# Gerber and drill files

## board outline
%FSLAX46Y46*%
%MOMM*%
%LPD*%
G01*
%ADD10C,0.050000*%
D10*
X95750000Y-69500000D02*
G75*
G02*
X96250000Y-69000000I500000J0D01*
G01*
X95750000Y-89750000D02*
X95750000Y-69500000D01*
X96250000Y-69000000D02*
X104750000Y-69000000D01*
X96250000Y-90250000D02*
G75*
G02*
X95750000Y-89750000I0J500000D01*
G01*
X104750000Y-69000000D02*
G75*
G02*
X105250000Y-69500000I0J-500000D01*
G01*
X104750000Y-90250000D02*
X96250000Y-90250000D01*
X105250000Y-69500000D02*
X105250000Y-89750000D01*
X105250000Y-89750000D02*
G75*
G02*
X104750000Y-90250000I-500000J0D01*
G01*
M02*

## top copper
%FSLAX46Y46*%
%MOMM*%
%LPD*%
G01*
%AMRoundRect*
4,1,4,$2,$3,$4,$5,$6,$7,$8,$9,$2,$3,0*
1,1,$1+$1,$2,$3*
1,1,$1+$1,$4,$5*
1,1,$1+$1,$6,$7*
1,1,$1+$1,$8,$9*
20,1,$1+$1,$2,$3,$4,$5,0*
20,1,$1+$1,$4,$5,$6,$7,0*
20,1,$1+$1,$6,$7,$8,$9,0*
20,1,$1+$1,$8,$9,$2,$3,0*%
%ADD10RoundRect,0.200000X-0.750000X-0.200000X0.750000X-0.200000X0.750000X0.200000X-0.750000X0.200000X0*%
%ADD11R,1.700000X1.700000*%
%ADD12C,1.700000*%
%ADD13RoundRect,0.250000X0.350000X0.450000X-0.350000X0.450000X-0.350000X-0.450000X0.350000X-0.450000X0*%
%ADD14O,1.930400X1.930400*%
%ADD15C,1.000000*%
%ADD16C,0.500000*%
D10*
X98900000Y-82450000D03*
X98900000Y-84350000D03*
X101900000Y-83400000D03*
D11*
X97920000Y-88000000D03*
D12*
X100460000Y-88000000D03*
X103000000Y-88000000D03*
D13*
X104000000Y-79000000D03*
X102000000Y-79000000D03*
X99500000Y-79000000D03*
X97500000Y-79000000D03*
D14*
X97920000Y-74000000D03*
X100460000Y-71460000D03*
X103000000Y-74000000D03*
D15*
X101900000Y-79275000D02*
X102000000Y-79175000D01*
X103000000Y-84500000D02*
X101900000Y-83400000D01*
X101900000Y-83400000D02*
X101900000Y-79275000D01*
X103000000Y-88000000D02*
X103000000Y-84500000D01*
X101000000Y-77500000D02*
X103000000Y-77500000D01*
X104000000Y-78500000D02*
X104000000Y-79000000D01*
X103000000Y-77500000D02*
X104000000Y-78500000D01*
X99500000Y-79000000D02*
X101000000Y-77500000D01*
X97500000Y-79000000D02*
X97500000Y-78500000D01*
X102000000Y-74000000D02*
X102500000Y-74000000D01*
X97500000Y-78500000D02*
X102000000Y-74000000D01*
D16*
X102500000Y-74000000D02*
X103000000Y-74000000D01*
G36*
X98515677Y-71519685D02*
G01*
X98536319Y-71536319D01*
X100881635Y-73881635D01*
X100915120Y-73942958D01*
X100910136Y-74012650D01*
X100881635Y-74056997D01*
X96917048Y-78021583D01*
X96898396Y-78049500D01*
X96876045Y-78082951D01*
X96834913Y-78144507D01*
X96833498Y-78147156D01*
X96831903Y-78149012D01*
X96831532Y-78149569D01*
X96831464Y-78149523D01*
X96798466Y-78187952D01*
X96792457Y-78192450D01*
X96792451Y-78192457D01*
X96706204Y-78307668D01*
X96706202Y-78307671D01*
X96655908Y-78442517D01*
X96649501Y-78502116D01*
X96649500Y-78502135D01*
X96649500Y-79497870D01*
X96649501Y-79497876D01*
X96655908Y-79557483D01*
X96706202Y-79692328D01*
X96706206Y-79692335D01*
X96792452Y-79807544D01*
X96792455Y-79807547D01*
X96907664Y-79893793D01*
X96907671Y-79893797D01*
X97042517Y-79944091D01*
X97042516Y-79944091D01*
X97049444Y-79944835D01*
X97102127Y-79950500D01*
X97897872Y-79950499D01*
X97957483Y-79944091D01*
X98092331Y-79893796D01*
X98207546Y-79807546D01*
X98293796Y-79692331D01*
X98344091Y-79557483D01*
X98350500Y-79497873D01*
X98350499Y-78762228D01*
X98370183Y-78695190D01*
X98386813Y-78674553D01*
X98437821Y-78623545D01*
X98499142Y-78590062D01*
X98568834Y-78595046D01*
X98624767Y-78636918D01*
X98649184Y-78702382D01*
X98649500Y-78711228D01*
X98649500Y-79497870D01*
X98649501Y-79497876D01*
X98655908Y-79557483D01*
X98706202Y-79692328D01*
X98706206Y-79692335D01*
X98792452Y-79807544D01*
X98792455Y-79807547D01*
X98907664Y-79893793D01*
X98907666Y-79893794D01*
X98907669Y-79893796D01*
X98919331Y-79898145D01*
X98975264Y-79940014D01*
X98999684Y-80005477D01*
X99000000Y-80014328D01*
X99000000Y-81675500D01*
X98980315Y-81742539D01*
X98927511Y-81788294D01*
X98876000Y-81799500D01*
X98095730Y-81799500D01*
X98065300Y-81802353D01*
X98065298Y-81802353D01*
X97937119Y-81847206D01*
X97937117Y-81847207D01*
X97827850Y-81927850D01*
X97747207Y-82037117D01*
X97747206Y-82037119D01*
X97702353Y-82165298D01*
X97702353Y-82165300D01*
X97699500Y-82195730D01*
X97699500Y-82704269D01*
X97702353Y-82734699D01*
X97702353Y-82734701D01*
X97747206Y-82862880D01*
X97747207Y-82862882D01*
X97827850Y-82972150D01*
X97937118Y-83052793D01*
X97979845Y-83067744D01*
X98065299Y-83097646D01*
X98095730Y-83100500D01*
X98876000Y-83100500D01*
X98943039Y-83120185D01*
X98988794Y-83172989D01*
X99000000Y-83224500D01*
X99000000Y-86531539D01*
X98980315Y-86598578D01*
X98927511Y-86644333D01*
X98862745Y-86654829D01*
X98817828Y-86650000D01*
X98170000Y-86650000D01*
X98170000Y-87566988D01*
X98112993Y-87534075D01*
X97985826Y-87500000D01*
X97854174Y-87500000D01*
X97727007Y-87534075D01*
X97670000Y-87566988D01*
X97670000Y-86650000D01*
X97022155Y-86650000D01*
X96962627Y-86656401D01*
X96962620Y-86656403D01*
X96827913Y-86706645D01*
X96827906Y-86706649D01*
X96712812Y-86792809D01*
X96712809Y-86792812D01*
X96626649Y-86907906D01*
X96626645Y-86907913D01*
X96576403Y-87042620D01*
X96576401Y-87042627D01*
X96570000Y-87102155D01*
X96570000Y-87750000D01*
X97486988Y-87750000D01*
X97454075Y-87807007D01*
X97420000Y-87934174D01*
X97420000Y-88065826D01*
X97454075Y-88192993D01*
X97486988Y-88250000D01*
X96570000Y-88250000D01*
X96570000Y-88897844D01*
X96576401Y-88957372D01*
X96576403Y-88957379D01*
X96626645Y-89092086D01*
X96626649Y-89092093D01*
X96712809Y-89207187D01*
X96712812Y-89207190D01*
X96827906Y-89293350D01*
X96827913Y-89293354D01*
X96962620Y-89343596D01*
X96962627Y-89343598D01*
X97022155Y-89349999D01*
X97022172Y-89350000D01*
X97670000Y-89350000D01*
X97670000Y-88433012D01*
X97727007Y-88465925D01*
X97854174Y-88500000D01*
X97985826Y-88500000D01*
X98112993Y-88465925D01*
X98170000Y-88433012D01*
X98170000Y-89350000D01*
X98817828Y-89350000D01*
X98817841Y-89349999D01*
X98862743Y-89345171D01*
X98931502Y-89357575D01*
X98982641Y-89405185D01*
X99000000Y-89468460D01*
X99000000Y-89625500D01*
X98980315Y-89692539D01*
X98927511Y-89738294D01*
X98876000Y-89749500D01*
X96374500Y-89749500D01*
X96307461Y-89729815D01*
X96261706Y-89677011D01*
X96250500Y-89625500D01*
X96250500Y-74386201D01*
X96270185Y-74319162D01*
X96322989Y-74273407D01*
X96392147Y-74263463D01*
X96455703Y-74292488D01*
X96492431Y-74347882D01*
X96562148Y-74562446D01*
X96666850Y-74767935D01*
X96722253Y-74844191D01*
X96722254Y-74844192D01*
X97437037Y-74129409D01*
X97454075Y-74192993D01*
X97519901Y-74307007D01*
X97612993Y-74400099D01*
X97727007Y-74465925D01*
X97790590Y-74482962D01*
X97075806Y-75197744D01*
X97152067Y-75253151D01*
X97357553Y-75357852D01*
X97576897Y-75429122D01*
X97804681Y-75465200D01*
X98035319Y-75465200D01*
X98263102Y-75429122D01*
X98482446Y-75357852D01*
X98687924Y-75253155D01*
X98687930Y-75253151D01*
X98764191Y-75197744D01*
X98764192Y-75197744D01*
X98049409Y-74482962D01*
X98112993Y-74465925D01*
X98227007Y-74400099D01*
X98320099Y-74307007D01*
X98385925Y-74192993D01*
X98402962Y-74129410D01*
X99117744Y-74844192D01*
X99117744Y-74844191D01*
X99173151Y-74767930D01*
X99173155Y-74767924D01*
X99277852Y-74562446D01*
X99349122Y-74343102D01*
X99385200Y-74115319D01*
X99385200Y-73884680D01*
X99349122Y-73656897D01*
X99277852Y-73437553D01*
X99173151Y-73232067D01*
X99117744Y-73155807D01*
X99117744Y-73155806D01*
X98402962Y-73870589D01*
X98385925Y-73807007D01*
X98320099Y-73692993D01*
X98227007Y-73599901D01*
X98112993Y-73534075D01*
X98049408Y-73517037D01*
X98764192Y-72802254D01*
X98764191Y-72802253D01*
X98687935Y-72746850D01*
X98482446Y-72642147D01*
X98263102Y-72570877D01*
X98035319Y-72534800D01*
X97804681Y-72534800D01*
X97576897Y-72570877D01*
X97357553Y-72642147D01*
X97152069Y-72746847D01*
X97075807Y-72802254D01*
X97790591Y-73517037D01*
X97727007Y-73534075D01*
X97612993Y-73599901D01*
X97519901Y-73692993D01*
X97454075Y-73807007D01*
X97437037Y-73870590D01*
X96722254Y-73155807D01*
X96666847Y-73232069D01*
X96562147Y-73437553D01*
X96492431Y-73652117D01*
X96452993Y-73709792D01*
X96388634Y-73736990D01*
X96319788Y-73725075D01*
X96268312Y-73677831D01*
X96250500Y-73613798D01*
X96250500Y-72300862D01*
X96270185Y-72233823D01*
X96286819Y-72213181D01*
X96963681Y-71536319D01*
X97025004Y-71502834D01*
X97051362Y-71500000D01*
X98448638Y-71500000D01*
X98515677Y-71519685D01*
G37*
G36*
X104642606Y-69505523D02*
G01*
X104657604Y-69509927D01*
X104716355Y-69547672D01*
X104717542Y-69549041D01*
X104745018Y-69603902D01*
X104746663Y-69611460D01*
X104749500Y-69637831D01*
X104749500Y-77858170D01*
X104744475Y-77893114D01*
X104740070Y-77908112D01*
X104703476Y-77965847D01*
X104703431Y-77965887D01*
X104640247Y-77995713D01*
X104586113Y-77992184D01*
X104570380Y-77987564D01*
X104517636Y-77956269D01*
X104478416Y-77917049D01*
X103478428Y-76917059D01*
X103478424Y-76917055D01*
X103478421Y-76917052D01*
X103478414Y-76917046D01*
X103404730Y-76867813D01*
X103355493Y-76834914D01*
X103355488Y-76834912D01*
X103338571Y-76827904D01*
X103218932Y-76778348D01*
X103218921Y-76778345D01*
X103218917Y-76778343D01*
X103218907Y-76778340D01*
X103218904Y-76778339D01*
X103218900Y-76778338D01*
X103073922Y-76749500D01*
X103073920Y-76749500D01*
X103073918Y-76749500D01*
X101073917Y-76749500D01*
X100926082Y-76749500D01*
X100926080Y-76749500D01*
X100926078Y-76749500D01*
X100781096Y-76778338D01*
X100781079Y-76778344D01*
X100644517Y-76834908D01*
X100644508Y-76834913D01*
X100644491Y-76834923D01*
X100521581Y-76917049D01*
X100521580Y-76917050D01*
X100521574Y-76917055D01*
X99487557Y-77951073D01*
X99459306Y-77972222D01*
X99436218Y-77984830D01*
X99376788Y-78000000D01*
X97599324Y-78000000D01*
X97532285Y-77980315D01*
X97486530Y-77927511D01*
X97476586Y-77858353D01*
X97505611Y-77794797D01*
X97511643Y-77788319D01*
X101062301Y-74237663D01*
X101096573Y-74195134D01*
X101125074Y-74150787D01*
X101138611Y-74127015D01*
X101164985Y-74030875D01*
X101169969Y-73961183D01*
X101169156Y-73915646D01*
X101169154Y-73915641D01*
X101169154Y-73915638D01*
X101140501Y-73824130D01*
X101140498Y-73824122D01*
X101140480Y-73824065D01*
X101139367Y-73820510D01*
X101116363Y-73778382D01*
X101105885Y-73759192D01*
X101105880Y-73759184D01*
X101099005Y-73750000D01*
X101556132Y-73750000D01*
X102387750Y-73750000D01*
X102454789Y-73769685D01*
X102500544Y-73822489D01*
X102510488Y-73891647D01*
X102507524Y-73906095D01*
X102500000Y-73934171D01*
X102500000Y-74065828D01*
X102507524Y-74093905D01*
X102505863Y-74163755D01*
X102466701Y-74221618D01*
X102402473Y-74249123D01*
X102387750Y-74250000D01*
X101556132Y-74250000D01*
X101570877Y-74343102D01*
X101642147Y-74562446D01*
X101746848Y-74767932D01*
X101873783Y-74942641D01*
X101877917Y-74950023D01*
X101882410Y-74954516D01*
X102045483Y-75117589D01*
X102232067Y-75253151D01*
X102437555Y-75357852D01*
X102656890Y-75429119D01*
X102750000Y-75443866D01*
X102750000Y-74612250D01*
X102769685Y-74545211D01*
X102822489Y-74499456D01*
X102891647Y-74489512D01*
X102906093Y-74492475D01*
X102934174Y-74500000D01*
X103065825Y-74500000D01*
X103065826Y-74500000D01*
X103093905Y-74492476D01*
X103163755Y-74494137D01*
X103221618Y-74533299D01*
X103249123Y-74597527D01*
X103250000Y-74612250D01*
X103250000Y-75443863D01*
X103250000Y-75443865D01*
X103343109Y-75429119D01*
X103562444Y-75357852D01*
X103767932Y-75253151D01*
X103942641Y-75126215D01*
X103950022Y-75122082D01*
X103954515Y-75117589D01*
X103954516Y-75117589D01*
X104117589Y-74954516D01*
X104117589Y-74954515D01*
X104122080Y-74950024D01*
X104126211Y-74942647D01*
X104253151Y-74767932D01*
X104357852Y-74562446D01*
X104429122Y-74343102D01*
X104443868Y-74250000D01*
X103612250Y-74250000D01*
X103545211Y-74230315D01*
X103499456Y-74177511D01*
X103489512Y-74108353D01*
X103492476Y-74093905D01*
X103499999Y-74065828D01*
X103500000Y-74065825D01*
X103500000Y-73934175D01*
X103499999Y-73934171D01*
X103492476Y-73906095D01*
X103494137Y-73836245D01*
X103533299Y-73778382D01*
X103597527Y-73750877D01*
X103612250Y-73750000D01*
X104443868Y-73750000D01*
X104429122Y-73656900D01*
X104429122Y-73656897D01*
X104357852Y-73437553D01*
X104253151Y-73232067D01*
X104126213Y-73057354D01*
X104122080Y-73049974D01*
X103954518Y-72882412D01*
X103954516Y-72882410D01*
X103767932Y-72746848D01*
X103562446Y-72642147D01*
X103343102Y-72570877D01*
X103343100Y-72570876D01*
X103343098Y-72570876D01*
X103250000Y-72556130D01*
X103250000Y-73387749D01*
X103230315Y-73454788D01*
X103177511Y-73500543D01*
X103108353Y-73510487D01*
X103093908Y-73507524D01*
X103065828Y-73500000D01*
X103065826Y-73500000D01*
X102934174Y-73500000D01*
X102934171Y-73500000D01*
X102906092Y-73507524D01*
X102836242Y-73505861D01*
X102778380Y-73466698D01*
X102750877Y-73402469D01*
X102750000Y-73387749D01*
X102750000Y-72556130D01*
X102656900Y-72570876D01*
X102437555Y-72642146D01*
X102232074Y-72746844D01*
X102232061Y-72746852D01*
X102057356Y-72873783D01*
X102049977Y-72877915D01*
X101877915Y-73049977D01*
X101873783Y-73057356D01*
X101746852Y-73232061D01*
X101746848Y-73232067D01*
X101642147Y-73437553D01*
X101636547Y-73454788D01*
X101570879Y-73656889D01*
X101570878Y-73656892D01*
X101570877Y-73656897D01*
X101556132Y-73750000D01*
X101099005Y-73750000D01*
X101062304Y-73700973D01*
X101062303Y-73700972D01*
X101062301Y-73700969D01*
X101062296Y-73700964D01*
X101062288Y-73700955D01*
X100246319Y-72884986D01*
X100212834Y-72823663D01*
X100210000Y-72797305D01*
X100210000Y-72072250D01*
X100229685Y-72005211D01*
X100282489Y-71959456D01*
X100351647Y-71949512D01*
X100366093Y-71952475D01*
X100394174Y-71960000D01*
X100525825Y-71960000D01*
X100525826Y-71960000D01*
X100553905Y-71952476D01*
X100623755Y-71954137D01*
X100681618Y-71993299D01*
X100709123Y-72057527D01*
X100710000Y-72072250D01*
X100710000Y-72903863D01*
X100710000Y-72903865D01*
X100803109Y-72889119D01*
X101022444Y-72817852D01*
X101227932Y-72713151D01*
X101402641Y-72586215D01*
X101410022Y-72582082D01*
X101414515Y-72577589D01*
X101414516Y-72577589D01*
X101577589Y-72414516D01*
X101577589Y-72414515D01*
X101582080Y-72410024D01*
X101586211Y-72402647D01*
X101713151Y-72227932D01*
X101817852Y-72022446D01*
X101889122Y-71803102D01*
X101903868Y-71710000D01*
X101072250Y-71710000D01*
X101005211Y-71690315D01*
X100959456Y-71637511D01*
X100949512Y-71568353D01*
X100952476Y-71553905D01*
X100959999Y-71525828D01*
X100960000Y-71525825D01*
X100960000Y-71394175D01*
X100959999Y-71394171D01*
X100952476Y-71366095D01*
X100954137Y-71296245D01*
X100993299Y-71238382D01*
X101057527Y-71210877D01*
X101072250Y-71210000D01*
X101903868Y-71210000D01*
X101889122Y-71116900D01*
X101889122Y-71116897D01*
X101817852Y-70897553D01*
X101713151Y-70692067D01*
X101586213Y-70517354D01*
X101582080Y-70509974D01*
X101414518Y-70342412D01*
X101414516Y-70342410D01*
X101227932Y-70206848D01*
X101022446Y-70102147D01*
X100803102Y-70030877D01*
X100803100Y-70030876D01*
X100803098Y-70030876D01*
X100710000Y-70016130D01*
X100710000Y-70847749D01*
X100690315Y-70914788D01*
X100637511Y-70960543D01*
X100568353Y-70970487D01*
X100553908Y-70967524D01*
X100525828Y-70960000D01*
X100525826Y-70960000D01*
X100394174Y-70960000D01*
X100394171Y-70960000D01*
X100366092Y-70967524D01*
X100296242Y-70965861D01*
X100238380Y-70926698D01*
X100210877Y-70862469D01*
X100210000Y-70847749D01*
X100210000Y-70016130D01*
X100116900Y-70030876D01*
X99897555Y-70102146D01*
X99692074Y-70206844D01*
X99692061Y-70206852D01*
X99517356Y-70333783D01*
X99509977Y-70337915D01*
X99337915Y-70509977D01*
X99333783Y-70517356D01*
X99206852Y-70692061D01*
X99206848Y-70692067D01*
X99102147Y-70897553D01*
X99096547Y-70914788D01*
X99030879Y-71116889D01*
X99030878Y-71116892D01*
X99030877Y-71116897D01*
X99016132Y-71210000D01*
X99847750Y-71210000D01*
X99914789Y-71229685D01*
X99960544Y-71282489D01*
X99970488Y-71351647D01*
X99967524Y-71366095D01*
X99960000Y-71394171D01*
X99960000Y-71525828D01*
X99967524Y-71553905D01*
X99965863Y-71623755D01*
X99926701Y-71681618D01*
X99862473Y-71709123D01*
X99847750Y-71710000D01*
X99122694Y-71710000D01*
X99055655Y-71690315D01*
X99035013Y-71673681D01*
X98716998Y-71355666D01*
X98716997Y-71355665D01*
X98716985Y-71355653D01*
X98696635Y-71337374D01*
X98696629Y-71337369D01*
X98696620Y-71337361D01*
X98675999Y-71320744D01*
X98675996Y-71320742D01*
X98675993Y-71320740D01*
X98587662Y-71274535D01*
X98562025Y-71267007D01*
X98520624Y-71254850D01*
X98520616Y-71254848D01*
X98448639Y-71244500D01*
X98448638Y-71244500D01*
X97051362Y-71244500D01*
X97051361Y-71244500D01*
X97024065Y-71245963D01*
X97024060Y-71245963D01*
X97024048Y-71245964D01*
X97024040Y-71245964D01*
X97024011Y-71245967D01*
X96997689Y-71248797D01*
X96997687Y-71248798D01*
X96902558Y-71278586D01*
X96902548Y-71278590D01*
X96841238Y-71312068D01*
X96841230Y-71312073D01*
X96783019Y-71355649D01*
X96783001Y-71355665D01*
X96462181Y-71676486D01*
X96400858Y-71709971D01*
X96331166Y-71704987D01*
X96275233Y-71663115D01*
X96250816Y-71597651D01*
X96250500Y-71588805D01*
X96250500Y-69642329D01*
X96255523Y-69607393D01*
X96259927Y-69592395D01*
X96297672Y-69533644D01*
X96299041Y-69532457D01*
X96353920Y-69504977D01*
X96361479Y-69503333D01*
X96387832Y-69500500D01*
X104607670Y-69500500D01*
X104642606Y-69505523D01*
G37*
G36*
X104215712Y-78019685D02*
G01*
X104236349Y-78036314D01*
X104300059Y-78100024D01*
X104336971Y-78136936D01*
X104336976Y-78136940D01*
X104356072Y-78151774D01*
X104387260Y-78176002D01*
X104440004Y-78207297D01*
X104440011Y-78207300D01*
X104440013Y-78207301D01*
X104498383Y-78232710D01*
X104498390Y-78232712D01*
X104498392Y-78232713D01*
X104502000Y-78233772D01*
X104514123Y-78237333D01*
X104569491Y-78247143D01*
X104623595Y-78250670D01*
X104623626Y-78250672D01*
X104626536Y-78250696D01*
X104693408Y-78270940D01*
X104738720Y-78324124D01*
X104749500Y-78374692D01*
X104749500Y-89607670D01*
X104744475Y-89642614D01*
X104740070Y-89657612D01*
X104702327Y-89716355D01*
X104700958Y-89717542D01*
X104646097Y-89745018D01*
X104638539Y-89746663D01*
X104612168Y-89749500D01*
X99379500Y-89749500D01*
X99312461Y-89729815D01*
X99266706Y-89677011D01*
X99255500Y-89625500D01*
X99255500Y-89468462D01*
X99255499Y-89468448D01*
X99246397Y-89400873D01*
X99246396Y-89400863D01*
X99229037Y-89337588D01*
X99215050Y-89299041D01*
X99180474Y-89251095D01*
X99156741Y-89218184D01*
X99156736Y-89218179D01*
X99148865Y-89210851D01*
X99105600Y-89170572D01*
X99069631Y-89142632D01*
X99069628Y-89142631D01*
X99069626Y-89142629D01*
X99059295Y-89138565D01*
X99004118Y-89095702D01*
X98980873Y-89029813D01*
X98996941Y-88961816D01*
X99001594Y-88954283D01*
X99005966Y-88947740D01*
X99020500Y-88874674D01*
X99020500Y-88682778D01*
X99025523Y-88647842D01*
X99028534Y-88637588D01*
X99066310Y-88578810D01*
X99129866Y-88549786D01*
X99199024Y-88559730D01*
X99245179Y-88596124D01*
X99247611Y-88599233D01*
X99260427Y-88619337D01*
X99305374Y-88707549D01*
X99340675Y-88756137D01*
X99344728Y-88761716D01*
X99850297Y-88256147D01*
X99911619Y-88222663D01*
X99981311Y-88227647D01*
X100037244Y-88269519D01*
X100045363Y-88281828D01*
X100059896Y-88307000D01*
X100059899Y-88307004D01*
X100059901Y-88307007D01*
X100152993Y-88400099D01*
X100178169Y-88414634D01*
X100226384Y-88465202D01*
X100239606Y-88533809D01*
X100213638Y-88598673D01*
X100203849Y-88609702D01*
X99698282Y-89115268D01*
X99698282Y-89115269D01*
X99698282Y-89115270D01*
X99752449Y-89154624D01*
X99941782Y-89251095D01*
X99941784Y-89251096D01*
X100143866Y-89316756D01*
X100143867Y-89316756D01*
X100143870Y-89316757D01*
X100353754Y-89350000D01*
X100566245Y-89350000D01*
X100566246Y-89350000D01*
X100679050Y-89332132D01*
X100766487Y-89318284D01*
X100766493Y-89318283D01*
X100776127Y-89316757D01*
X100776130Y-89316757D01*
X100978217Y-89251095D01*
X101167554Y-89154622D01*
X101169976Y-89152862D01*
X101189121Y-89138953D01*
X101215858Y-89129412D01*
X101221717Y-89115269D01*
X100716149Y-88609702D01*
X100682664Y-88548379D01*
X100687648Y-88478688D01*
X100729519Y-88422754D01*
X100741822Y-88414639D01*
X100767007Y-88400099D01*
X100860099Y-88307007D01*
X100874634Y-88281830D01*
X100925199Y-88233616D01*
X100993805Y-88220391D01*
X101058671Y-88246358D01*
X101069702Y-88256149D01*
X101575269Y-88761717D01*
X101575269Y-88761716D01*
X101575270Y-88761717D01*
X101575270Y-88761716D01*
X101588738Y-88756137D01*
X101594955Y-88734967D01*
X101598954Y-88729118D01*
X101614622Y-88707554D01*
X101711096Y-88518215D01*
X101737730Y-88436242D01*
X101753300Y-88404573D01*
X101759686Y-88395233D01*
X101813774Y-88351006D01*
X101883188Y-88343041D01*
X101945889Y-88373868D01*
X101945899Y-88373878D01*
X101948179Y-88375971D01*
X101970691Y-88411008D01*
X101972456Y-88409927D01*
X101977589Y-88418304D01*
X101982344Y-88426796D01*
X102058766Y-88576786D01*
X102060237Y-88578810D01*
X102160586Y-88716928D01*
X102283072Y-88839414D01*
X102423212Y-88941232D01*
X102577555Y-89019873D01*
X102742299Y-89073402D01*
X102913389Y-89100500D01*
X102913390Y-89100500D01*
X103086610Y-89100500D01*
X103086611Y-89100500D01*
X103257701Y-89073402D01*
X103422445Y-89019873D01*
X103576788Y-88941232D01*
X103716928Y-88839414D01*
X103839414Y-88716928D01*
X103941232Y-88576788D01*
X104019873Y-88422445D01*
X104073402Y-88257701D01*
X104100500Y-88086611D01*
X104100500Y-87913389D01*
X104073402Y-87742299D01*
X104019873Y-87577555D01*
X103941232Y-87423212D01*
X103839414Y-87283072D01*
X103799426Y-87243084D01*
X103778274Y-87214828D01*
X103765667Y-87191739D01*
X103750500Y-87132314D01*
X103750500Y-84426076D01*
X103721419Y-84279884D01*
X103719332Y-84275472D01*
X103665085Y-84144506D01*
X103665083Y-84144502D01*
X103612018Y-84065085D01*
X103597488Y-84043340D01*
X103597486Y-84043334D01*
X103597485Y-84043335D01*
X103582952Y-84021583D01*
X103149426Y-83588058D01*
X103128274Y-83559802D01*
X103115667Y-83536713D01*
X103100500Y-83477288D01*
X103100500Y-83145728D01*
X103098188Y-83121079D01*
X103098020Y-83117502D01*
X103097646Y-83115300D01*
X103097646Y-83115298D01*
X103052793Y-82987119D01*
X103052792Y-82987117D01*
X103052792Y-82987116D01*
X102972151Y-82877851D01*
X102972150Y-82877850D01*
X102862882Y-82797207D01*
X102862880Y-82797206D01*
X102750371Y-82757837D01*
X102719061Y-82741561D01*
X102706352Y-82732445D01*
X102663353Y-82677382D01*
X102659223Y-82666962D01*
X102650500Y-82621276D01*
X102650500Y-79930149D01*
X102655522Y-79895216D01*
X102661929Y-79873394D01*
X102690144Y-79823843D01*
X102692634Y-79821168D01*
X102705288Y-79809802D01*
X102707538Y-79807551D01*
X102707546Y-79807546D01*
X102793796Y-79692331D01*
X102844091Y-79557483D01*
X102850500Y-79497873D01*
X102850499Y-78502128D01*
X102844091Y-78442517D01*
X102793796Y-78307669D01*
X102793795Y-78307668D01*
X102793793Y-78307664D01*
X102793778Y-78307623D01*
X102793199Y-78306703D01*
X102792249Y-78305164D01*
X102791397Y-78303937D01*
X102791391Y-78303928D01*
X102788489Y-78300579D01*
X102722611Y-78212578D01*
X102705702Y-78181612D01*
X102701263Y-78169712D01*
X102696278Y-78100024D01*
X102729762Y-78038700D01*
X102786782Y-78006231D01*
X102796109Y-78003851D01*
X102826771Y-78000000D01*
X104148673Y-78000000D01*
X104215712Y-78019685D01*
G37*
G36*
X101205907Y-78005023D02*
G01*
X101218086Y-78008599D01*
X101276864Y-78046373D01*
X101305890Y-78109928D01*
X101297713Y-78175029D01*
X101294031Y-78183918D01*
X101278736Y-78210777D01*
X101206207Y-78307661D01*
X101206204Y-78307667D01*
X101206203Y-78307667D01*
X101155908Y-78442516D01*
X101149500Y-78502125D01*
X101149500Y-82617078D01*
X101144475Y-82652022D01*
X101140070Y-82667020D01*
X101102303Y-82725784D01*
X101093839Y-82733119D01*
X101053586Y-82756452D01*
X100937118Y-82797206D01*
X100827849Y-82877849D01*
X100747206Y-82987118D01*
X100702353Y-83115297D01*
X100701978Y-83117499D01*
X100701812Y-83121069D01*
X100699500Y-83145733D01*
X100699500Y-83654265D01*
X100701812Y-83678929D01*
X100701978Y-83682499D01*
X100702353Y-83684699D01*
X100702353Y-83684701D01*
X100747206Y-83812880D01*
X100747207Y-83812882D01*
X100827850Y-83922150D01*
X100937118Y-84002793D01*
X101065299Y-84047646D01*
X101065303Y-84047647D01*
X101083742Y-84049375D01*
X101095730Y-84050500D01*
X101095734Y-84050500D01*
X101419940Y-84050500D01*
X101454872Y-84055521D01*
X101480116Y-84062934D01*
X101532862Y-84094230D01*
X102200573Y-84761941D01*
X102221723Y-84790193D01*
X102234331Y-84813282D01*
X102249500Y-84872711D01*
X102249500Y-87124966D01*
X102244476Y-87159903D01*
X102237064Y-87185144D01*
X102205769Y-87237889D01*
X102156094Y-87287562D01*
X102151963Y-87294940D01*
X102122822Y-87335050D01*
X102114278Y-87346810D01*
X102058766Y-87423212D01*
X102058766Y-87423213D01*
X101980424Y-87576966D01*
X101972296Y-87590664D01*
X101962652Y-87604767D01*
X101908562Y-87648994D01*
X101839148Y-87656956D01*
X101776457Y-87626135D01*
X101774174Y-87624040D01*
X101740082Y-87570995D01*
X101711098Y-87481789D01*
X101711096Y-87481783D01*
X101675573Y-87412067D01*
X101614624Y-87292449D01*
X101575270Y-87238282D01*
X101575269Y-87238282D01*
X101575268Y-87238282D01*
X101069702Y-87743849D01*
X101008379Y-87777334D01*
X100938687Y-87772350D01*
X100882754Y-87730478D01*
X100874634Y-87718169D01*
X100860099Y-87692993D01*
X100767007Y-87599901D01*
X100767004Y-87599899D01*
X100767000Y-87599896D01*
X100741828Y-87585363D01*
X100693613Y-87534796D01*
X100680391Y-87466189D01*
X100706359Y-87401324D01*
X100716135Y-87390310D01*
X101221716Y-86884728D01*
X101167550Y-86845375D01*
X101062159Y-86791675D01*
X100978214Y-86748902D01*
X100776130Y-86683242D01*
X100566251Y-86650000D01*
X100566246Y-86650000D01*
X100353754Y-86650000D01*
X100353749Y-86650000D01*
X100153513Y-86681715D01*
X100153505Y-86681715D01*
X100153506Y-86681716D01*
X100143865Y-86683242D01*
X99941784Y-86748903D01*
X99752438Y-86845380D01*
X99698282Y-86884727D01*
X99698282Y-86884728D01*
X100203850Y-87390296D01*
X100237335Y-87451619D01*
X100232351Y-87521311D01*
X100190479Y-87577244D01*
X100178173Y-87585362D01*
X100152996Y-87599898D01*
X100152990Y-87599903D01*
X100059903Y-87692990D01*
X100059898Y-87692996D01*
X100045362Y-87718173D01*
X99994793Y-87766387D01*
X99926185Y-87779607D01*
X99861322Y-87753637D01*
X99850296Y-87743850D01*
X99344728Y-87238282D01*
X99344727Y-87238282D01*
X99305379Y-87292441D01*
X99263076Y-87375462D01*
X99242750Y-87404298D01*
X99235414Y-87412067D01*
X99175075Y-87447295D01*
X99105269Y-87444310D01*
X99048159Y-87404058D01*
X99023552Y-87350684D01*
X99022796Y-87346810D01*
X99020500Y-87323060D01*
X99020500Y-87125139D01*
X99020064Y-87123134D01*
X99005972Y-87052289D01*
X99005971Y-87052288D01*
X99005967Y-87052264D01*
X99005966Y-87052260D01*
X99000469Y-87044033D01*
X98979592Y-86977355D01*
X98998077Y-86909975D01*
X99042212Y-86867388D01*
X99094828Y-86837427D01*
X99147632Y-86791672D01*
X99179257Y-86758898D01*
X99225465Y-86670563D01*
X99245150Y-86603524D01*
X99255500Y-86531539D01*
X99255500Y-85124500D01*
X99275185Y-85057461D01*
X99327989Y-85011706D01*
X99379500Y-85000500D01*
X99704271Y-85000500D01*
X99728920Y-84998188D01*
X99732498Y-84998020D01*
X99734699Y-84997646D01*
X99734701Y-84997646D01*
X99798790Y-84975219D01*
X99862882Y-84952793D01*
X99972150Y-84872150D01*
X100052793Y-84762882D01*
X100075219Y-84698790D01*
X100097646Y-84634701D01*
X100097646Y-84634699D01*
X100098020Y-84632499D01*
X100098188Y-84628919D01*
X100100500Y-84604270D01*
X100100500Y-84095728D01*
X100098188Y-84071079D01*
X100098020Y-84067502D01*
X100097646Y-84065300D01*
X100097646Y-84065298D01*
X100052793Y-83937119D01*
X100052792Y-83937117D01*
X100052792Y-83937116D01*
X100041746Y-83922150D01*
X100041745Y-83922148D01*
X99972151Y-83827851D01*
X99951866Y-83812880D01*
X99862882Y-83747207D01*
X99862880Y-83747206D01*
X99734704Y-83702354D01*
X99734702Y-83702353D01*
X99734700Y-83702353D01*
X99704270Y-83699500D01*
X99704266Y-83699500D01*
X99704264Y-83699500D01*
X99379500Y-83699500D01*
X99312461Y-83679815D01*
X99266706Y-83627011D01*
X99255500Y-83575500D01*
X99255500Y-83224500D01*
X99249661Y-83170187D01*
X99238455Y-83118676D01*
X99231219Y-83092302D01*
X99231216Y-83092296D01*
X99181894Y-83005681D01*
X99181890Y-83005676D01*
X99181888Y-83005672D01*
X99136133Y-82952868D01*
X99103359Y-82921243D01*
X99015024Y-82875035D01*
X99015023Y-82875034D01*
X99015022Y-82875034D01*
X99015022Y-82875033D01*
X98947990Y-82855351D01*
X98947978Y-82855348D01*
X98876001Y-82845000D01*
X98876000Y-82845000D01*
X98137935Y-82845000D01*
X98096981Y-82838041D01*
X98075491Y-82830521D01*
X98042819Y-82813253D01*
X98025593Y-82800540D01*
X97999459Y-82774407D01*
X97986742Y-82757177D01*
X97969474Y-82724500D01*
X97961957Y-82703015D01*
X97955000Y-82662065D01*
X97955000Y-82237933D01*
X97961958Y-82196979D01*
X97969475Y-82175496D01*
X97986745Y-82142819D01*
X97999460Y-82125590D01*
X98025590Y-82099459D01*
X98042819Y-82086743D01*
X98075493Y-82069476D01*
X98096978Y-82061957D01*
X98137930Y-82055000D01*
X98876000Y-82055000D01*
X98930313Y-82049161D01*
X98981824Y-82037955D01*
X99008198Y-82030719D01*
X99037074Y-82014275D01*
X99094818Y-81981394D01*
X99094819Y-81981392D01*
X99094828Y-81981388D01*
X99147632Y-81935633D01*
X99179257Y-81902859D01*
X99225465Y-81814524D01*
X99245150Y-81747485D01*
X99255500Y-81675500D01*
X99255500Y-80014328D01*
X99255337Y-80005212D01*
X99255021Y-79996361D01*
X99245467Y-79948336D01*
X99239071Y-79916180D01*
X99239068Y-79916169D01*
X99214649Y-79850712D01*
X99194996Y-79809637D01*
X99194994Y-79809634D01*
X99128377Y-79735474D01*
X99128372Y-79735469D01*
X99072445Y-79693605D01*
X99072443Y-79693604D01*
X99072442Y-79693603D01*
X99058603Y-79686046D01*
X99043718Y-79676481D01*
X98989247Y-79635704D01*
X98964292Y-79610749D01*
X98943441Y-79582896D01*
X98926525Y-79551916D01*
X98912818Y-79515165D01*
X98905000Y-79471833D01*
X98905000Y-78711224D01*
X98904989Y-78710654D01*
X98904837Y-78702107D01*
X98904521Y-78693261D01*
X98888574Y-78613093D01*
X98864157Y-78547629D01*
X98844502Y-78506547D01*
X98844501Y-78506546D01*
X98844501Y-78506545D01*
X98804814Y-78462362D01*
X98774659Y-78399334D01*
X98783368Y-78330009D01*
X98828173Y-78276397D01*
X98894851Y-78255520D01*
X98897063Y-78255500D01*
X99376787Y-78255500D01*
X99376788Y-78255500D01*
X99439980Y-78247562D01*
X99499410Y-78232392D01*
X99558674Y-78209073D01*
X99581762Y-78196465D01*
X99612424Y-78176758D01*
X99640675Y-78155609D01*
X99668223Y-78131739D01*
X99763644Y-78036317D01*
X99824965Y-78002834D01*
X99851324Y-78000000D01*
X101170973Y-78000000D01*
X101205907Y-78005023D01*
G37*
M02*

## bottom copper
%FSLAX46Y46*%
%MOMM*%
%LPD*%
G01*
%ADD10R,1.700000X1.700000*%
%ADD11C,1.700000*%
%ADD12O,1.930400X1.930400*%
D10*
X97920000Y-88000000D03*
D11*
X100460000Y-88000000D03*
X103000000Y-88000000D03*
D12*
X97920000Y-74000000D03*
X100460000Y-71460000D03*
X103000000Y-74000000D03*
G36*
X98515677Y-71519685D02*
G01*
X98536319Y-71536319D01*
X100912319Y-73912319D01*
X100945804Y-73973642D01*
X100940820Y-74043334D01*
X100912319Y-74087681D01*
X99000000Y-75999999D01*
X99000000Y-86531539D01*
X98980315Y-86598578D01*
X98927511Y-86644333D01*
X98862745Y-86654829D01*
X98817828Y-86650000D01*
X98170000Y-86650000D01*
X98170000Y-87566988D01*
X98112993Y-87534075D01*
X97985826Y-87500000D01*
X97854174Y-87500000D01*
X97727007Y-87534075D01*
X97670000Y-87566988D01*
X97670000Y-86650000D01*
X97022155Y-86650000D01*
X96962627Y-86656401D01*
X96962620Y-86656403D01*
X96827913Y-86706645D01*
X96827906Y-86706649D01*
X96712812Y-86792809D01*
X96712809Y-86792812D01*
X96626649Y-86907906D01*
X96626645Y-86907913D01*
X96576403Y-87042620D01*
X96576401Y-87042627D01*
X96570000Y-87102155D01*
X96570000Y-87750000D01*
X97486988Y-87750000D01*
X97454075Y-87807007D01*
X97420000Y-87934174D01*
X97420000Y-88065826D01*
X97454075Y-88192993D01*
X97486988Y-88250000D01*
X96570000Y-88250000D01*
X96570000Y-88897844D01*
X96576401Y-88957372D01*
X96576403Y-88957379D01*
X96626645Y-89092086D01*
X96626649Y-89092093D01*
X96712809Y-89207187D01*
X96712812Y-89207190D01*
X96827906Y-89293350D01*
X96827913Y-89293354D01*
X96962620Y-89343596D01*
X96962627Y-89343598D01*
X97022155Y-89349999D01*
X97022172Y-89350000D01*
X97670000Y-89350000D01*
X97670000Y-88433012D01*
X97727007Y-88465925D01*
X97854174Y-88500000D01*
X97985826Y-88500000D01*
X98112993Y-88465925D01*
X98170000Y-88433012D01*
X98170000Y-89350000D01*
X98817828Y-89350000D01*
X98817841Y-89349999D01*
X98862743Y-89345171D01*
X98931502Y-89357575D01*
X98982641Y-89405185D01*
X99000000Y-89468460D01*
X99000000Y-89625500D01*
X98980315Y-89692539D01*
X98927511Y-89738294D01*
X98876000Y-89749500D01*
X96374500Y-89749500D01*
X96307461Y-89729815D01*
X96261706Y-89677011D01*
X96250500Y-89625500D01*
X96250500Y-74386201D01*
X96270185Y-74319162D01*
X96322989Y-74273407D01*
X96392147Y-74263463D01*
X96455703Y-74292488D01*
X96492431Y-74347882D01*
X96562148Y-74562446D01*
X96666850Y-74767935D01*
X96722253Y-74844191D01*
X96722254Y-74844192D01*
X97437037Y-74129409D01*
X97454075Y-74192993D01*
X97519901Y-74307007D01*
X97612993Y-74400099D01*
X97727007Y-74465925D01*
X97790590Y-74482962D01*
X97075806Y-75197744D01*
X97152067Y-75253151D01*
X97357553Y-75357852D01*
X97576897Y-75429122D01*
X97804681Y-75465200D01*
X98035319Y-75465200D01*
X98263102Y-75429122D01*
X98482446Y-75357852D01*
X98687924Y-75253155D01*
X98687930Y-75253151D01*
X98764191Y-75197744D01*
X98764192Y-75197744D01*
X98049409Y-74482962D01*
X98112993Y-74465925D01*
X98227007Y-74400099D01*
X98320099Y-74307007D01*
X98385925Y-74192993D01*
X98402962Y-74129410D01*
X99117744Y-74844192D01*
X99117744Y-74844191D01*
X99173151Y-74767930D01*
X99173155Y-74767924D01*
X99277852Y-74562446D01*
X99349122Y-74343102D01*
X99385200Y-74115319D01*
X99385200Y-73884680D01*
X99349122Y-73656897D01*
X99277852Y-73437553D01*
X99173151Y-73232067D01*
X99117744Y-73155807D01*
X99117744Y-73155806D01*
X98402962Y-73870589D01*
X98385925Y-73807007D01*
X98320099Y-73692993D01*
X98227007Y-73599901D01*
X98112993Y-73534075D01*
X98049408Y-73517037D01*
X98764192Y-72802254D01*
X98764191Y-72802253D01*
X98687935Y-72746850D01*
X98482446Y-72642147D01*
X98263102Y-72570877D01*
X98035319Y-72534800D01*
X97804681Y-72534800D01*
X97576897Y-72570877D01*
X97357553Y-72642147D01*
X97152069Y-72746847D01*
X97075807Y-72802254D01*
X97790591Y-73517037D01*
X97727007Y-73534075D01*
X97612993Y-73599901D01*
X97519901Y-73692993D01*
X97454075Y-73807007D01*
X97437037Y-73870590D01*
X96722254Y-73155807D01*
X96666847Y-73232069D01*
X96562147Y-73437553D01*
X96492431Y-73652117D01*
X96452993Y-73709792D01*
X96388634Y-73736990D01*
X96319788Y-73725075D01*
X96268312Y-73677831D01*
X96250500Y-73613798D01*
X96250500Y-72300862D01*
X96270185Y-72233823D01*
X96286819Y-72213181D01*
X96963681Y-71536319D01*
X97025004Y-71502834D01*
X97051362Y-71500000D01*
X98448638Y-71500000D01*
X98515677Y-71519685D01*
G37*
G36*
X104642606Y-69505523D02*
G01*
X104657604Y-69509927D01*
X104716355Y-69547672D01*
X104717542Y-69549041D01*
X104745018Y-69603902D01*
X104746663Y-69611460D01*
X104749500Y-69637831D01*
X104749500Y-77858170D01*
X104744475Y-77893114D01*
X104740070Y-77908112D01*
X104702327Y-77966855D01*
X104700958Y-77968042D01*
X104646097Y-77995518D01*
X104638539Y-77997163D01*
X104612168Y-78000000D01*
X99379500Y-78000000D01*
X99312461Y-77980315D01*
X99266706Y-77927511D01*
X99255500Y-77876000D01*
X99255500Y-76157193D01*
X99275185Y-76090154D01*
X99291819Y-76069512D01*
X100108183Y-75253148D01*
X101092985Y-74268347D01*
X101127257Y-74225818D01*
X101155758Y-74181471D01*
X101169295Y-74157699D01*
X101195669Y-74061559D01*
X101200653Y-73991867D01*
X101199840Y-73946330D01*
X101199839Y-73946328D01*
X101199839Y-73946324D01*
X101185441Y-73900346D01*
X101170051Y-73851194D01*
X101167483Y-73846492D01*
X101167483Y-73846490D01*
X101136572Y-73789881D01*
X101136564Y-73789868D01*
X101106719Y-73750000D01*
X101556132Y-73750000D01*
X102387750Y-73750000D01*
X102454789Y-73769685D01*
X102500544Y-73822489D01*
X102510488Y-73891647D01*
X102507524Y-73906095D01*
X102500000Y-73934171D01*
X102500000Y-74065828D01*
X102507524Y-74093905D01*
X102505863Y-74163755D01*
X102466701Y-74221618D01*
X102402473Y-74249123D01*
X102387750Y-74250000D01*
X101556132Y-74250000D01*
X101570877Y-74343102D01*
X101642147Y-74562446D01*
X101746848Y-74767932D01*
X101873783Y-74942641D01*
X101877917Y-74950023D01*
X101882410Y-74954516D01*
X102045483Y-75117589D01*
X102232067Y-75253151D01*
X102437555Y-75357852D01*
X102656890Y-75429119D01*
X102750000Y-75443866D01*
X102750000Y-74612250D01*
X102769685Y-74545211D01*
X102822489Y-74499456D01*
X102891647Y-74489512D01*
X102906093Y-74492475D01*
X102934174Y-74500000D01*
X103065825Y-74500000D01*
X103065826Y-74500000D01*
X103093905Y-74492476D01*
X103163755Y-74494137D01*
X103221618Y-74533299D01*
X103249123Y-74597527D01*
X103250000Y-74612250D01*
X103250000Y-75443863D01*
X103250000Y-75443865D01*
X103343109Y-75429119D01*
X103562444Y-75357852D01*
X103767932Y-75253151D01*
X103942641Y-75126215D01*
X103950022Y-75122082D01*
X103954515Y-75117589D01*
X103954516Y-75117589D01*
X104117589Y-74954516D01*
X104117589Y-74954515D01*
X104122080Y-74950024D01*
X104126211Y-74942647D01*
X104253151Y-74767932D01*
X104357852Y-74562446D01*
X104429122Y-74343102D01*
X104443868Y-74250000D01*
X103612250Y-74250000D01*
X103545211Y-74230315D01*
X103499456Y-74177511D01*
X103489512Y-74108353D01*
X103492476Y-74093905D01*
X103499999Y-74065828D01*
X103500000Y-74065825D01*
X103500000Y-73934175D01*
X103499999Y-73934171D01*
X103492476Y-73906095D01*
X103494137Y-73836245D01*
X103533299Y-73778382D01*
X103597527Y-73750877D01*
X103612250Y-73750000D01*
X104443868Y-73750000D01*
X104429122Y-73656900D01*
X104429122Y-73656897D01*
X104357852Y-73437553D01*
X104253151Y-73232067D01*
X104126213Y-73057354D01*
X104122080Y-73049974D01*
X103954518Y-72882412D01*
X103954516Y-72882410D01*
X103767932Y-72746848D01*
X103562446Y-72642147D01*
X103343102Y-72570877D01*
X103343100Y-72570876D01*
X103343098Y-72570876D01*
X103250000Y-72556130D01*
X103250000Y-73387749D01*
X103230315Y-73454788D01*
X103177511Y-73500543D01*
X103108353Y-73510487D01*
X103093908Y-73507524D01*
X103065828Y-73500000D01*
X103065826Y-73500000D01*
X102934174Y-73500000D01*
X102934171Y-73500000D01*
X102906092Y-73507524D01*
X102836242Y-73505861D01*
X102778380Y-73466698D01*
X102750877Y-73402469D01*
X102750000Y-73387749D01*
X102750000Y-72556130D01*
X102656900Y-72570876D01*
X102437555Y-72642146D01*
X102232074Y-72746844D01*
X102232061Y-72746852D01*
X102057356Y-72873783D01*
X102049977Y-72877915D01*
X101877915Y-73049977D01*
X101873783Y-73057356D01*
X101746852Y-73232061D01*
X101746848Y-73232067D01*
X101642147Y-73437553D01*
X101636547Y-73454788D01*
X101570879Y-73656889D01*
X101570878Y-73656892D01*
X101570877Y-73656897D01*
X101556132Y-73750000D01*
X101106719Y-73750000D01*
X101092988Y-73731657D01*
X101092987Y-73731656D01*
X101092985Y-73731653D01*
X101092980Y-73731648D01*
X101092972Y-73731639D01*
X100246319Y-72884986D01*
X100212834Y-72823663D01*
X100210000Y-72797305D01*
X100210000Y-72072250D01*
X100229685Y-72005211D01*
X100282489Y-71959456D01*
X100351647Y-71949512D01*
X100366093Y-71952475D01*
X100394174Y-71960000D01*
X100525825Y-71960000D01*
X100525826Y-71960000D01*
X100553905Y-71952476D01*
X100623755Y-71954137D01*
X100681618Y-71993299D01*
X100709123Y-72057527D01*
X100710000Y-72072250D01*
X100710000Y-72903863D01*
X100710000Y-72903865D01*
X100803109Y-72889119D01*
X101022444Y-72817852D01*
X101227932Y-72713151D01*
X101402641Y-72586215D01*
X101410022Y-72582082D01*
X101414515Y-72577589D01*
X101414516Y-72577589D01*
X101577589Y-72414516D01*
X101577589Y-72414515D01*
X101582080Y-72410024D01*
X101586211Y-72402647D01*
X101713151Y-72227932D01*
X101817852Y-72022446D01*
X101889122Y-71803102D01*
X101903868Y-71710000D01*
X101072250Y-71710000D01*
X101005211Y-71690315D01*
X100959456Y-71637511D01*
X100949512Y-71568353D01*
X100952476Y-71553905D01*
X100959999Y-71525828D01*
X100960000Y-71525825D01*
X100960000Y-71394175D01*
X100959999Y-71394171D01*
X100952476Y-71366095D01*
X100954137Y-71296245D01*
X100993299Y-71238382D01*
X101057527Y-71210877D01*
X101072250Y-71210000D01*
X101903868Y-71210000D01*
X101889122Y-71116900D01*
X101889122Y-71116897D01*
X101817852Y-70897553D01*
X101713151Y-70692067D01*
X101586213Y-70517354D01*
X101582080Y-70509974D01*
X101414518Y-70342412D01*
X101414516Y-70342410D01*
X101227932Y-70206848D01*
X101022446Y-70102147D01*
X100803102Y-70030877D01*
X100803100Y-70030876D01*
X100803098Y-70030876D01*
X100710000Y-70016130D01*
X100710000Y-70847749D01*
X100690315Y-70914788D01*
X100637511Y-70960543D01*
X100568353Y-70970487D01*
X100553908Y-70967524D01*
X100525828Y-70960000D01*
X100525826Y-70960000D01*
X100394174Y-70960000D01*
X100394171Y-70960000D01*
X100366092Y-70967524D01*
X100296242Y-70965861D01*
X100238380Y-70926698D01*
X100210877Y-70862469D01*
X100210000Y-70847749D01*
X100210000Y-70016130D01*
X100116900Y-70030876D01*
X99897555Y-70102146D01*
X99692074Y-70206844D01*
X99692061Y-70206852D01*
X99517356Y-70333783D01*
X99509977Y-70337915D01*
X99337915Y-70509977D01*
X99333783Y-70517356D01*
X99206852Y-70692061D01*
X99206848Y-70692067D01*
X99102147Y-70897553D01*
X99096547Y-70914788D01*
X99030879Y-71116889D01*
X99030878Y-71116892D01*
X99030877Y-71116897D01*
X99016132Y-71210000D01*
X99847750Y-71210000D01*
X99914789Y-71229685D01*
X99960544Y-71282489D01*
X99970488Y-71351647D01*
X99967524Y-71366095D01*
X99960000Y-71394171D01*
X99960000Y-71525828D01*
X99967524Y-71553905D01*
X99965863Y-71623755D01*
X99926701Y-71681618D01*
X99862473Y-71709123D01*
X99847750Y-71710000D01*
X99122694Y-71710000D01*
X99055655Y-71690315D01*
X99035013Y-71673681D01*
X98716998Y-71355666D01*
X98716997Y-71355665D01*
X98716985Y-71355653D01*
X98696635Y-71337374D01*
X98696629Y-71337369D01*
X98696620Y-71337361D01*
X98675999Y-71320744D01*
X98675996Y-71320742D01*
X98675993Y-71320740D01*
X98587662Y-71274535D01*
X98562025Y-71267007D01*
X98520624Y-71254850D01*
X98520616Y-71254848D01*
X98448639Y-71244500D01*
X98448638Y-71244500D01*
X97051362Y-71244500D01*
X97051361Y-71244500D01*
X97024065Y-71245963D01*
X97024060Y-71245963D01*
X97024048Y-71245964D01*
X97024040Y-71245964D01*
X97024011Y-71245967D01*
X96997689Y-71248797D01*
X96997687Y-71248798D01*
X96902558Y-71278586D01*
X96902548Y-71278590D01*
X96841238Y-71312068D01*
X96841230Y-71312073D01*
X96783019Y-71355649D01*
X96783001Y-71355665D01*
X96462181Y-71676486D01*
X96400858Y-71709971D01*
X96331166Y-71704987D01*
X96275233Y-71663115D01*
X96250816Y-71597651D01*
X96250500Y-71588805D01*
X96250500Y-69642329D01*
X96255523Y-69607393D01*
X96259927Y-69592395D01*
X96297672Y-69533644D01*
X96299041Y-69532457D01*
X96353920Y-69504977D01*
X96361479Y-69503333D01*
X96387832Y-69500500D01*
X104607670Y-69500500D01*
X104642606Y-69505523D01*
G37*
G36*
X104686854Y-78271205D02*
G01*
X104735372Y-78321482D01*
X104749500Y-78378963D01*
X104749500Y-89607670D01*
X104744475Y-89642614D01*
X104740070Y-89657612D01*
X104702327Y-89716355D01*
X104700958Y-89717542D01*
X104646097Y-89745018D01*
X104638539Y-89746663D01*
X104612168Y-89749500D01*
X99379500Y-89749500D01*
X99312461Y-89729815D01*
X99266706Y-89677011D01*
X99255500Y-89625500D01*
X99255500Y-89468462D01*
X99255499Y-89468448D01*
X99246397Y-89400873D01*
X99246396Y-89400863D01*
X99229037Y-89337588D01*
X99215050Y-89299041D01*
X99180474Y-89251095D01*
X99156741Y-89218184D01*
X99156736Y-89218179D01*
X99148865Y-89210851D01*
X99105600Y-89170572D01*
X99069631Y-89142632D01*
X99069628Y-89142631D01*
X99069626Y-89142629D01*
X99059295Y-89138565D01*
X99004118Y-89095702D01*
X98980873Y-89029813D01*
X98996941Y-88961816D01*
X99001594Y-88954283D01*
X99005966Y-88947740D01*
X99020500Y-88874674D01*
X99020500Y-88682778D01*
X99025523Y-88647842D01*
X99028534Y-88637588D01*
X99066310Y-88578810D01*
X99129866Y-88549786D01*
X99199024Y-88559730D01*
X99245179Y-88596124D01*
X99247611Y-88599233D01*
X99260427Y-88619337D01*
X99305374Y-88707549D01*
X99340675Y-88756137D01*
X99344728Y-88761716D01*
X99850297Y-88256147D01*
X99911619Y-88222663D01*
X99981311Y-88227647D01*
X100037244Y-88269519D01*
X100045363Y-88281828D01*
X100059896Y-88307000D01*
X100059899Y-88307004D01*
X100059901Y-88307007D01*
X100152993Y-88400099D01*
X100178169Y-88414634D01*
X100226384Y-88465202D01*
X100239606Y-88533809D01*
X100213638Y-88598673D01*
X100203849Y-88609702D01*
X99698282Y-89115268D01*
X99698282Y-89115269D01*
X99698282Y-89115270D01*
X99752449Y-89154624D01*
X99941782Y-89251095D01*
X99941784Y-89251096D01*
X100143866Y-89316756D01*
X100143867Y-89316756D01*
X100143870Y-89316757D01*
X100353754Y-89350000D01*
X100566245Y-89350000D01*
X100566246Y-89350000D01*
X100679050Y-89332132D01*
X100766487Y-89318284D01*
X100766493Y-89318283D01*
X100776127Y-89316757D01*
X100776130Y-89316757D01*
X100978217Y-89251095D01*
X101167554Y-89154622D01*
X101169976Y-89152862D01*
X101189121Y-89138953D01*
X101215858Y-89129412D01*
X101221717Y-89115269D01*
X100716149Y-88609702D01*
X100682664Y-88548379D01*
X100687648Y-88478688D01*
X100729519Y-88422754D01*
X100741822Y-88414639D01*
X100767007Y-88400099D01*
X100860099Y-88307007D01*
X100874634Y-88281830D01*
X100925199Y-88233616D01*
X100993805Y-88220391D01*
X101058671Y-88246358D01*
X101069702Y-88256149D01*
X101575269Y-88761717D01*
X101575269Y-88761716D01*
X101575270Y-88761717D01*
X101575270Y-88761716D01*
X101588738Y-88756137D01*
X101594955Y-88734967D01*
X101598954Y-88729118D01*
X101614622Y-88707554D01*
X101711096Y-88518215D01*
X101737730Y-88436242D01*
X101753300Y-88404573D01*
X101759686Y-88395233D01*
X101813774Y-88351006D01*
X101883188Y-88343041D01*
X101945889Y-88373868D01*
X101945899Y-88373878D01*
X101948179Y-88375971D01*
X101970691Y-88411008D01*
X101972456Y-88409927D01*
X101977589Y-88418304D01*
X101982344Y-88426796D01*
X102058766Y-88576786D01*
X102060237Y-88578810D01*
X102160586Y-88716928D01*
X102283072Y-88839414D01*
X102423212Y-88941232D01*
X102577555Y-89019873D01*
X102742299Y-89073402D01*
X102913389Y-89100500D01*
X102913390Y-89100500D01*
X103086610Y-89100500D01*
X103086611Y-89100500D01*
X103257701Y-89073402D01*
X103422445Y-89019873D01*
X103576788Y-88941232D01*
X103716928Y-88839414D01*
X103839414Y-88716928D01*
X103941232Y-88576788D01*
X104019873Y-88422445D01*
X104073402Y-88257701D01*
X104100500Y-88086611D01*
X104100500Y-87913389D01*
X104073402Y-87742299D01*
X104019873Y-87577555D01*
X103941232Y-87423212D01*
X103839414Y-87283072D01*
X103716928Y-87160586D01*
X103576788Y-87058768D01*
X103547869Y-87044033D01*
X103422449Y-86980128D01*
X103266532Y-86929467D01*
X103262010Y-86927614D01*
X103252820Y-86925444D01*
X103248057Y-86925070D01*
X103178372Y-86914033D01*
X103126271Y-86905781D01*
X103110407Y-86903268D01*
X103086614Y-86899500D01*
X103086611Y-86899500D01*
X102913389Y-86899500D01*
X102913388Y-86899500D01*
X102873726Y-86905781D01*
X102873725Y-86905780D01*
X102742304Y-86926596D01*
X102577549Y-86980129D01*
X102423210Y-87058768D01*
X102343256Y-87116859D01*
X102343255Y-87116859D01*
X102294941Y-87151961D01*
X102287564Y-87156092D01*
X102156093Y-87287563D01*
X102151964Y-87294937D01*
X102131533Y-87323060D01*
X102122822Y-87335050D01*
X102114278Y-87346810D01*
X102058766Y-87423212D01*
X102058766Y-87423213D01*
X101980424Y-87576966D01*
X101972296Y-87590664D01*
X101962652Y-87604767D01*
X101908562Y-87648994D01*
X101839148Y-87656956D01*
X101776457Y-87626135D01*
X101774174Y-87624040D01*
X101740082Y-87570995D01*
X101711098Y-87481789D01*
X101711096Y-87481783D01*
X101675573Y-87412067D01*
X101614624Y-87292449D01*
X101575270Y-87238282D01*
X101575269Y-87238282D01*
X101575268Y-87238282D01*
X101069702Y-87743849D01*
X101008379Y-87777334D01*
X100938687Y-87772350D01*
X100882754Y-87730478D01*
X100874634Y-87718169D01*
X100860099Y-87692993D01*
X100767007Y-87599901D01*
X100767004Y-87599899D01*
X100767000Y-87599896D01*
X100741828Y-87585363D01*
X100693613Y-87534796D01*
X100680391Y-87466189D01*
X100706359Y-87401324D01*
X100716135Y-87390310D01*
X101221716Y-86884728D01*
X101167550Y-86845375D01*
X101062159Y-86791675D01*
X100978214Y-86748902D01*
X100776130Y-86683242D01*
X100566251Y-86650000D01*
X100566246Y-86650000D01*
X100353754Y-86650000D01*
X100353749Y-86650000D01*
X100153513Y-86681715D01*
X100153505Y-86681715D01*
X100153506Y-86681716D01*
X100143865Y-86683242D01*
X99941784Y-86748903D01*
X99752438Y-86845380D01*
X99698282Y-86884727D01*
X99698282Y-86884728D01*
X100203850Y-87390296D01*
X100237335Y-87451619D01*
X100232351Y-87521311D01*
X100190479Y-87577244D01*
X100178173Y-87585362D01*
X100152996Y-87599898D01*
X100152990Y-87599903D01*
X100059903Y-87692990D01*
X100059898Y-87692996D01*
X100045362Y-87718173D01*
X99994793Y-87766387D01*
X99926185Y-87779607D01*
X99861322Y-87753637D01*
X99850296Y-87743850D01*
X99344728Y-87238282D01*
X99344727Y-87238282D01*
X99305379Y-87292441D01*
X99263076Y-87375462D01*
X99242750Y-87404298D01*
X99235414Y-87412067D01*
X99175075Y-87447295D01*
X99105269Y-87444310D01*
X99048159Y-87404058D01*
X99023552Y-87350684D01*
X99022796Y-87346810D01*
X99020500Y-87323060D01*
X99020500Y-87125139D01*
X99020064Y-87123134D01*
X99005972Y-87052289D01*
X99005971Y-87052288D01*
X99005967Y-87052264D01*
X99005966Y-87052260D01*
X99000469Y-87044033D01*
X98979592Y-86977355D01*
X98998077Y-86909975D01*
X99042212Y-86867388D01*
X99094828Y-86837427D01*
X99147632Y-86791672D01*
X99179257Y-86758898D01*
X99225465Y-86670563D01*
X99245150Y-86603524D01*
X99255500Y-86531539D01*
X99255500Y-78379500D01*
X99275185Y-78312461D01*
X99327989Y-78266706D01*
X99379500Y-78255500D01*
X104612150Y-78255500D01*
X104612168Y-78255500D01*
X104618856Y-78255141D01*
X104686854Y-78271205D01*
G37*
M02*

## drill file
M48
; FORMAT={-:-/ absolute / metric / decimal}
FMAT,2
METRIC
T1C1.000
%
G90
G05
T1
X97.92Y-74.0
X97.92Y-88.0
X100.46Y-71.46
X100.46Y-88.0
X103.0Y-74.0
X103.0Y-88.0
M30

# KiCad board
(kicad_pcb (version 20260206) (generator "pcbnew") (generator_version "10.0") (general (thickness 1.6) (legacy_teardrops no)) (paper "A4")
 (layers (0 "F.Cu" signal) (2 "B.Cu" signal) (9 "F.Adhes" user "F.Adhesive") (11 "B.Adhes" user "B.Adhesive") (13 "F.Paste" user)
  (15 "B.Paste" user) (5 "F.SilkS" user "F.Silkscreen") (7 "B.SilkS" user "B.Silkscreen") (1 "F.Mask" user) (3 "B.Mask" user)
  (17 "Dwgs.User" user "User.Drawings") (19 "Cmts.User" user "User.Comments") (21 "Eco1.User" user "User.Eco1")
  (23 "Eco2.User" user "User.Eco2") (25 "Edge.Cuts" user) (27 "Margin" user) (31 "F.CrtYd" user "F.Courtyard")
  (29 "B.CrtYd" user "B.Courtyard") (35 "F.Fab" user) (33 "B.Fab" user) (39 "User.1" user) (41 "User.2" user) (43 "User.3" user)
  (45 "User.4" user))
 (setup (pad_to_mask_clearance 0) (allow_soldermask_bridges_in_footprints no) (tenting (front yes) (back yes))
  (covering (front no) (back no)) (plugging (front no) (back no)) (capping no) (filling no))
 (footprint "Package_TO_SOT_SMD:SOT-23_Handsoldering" (layer "F.Cu") (at 100.4 83.4)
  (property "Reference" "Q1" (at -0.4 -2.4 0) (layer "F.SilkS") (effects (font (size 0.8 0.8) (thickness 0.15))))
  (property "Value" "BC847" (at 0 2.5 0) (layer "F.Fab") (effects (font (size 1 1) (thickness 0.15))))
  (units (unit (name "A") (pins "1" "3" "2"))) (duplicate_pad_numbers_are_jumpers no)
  (pad "1" smd roundrect (at -1.5 -0.95) (size 1.9 0.8) (layers "F.Cu" "F.Mask" "F.Paste") (roundrect_rratio 0.25) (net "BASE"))
  (pad "2" smd roundrect (at -1.5 0.95) (size 1.9 0.8) (layers "F.Cu" "F.Mask" "F.Paste") (roundrect_rratio 0.25) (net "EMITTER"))
  (pad "3" smd roundrect (at 1.5 0) (size 1.9 0.8) (layers "F.Cu" "F.Mask" "F.Paste") (roundrect_rratio 0.25) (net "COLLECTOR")))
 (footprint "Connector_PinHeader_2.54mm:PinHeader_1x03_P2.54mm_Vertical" (layer "F.Cu") (at 97.92 88 90)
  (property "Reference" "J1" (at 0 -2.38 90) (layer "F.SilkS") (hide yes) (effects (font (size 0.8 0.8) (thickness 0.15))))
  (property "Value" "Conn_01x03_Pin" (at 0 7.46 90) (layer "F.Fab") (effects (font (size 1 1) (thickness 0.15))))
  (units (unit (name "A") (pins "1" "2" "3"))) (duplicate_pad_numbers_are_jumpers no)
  (pad "1" thru_hole rect (at 0 0 90) (size 1.7 1.7) (drill 1) (layers "*.Cu" "*.Mask") (remove_unused_layers no) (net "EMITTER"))
  (pad "2" thru_hole circle (at 0 2.54 90) (size 1.7 1.7) (drill 1) (layers "*.Cu" "*.Mask") (remove_unused_layers no) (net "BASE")
   (zone_connect 1))
  (pad "3" thru_hole circle (at 0 5.08 90) (size 1.7 1.7) (drill 1) (layers "*.Cu" "*.Mask") (remove_unused_layers no) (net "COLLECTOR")
   (zone_connect 1)))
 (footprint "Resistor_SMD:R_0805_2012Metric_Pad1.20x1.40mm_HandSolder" (layer "F.Cu") (at 103 79 180)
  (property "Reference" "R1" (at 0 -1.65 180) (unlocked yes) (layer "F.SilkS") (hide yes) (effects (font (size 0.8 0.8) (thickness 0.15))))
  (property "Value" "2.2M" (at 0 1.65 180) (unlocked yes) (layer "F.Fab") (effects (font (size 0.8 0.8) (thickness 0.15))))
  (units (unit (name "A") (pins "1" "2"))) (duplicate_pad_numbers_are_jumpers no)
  (pad "1" smd roundrect (at -1 0 180) (size 1.2 1.4) (layers "F.Cu" "F.Mask" "F.Paste") (roundrect_rratio 0.208333) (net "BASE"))
  (pad "2" smd roundrect (at 1 0 180) (size 1.2 1.4) (layers "F.Cu" "F.Mask" "F.Paste") (roundrect_rratio 0.208333) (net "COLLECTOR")))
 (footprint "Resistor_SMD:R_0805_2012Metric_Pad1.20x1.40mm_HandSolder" (layer "F.Cu") (at 98.5 79 180)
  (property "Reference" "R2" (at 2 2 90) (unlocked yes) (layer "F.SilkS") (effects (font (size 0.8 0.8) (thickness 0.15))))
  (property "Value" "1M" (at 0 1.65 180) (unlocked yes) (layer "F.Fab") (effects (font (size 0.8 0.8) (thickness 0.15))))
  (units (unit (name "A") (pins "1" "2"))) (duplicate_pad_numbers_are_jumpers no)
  (pad "1" smd roundrect (at -1 0 180) (size 1.2 1.4) (layers "F.Cu" "F.Mask" "F.Paste") (roundrect_rratio 0.208333) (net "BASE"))
  (pad "2" smd roundrect (at 1 0 180) (size 1.2 1.4) (layers "F.Cu" "F.Mask" "F.Paste") (roundrect_rratio 0.208333) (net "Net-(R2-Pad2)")))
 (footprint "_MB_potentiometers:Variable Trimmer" (layer "F.Cu") (at 100.46 74)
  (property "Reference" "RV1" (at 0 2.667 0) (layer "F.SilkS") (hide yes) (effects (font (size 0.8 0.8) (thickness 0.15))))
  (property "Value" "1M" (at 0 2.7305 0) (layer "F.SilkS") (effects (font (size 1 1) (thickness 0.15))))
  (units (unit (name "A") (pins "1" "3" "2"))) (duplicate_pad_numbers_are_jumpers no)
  (pad "1" thru_hole oval (at -2.54 0) (size 1.9304 1.9304) (drill 1) (layers "*.Cu" "*.Mask") (remove_unused_layers no) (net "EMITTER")
   (thermal_bridge_angle 45))
  (pad "2" thru_hole oval (at 0 -2.54) (size 1.9304 1.9304) (drill 1) (layers "*.Cu" "*.Mask") (remove_unused_layers no)
   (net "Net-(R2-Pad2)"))
  (pad "3" thru_hole oval (at 2.54 0) (size 1.9304 1.9304) (drill 1) (layers "*.Cu" "*.Mask") (remove_unused_layers no)
   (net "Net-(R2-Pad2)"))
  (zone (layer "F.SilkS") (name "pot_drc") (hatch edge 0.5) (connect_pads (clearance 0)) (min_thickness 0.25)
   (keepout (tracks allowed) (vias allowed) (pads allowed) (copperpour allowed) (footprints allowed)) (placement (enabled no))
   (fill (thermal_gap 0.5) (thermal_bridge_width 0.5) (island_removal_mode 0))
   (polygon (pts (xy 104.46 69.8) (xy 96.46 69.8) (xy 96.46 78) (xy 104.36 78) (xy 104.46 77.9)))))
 (gr_arc (start 95.75 69.5) (mid 95.896447 69.146447) (end 96.25 69) (stroke (width 0.05) (type default)) (layer "Edge.Cuts"))
 (gr_line (start 95.75 89.75) (end 95.75 69.5) (stroke (width 0.05) (type default)) (layer "Edge.Cuts"))
 (gr_line (start 96.25 69) (end 104.75 69) (stroke (width 0.05) (type default)) (layer "Edge.Cuts"))
 (gr_arc (start 96.25 90.25) (mid 95.896447 90.103553) (end 95.75 89.75) (stroke (width 0.05) (type default)) (layer "Edge.Cuts"))
 (gr_arc (start 104.75 69) (mid 105.103553 69.146447) (end 105.25 69.5) (stroke (width 0.05) (type default)) (layer "Edge.Cuts"))
 (gr_line (start 104.75 90.25) (end 96.25 90.25) (stroke (width 0.05) (type default)) (layer "Edge.Cuts"))
 (gr_line (start 105.25 69.5) (end 105.25 89.75) (stroke (width 0.05) (type default)) (layer "Edge.Cuts"))
 (gr_arc (start 105.25 89.75) (mid 105.103553 90.103553) (end 104.75 90.25) (stroke (width 0.05) (type default)) (layer "Edge.Cuts"))
 (segment (start 101.9 79.275) (end 102 79.175) (width 1) (layer "F.Cu") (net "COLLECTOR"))
 (segment (start 103 84.5) (end 101.9 83.4) (width 1) (layer "F.Cu") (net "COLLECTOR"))
 (segment (start 101.9 83.4) (end 101.9 79.275) (width 1) (layer "F.Cu") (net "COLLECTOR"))
 (segment (start 103 88) (end 103 84.5) (width 1) (layer "F.Cu") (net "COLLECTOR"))
 (segment (start 101 77.5) (end 103 77.5) (width 1) (layer "F.Cu") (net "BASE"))
 (segment (start 104 78.5) (end 104 79) (width 1) (layer "F.Cu") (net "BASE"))
 (segment (start 103 77.5) (end 104 78.5) (width 1) (layer "F.Cu") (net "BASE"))
 (segment (start 99.5 79) (end 101 77.5) (width 1) (layer "F.Cu") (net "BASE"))
 (segment (start 97.5 79) (end 97.5 78.5) (width 1) (layer "F.Cu") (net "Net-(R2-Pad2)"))
 (segment (start 102 74) (end 102.5 74) (width 1) (layer "F.Cu") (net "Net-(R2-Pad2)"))
 (segment (start 97.5 78.5) (end 102 74) (width 1) (layer "F.Cu") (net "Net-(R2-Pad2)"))
 (segment (start 102.5 74) (end 103 74) (width 0.5) (layer "F.Cu") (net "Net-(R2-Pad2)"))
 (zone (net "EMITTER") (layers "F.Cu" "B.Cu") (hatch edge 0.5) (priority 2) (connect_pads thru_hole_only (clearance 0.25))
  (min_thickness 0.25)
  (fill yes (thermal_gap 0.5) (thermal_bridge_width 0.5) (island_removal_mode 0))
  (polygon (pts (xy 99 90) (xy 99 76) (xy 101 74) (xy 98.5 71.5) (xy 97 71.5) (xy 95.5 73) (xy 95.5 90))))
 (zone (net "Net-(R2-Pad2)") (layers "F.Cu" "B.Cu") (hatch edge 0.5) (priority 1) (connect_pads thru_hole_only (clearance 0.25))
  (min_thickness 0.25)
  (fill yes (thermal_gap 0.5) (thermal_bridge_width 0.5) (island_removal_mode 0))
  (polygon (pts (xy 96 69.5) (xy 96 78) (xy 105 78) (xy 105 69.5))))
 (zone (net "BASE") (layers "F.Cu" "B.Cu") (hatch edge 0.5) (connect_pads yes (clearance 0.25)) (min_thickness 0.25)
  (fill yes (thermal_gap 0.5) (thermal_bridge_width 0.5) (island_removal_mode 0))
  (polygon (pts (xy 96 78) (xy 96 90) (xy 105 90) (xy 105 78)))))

